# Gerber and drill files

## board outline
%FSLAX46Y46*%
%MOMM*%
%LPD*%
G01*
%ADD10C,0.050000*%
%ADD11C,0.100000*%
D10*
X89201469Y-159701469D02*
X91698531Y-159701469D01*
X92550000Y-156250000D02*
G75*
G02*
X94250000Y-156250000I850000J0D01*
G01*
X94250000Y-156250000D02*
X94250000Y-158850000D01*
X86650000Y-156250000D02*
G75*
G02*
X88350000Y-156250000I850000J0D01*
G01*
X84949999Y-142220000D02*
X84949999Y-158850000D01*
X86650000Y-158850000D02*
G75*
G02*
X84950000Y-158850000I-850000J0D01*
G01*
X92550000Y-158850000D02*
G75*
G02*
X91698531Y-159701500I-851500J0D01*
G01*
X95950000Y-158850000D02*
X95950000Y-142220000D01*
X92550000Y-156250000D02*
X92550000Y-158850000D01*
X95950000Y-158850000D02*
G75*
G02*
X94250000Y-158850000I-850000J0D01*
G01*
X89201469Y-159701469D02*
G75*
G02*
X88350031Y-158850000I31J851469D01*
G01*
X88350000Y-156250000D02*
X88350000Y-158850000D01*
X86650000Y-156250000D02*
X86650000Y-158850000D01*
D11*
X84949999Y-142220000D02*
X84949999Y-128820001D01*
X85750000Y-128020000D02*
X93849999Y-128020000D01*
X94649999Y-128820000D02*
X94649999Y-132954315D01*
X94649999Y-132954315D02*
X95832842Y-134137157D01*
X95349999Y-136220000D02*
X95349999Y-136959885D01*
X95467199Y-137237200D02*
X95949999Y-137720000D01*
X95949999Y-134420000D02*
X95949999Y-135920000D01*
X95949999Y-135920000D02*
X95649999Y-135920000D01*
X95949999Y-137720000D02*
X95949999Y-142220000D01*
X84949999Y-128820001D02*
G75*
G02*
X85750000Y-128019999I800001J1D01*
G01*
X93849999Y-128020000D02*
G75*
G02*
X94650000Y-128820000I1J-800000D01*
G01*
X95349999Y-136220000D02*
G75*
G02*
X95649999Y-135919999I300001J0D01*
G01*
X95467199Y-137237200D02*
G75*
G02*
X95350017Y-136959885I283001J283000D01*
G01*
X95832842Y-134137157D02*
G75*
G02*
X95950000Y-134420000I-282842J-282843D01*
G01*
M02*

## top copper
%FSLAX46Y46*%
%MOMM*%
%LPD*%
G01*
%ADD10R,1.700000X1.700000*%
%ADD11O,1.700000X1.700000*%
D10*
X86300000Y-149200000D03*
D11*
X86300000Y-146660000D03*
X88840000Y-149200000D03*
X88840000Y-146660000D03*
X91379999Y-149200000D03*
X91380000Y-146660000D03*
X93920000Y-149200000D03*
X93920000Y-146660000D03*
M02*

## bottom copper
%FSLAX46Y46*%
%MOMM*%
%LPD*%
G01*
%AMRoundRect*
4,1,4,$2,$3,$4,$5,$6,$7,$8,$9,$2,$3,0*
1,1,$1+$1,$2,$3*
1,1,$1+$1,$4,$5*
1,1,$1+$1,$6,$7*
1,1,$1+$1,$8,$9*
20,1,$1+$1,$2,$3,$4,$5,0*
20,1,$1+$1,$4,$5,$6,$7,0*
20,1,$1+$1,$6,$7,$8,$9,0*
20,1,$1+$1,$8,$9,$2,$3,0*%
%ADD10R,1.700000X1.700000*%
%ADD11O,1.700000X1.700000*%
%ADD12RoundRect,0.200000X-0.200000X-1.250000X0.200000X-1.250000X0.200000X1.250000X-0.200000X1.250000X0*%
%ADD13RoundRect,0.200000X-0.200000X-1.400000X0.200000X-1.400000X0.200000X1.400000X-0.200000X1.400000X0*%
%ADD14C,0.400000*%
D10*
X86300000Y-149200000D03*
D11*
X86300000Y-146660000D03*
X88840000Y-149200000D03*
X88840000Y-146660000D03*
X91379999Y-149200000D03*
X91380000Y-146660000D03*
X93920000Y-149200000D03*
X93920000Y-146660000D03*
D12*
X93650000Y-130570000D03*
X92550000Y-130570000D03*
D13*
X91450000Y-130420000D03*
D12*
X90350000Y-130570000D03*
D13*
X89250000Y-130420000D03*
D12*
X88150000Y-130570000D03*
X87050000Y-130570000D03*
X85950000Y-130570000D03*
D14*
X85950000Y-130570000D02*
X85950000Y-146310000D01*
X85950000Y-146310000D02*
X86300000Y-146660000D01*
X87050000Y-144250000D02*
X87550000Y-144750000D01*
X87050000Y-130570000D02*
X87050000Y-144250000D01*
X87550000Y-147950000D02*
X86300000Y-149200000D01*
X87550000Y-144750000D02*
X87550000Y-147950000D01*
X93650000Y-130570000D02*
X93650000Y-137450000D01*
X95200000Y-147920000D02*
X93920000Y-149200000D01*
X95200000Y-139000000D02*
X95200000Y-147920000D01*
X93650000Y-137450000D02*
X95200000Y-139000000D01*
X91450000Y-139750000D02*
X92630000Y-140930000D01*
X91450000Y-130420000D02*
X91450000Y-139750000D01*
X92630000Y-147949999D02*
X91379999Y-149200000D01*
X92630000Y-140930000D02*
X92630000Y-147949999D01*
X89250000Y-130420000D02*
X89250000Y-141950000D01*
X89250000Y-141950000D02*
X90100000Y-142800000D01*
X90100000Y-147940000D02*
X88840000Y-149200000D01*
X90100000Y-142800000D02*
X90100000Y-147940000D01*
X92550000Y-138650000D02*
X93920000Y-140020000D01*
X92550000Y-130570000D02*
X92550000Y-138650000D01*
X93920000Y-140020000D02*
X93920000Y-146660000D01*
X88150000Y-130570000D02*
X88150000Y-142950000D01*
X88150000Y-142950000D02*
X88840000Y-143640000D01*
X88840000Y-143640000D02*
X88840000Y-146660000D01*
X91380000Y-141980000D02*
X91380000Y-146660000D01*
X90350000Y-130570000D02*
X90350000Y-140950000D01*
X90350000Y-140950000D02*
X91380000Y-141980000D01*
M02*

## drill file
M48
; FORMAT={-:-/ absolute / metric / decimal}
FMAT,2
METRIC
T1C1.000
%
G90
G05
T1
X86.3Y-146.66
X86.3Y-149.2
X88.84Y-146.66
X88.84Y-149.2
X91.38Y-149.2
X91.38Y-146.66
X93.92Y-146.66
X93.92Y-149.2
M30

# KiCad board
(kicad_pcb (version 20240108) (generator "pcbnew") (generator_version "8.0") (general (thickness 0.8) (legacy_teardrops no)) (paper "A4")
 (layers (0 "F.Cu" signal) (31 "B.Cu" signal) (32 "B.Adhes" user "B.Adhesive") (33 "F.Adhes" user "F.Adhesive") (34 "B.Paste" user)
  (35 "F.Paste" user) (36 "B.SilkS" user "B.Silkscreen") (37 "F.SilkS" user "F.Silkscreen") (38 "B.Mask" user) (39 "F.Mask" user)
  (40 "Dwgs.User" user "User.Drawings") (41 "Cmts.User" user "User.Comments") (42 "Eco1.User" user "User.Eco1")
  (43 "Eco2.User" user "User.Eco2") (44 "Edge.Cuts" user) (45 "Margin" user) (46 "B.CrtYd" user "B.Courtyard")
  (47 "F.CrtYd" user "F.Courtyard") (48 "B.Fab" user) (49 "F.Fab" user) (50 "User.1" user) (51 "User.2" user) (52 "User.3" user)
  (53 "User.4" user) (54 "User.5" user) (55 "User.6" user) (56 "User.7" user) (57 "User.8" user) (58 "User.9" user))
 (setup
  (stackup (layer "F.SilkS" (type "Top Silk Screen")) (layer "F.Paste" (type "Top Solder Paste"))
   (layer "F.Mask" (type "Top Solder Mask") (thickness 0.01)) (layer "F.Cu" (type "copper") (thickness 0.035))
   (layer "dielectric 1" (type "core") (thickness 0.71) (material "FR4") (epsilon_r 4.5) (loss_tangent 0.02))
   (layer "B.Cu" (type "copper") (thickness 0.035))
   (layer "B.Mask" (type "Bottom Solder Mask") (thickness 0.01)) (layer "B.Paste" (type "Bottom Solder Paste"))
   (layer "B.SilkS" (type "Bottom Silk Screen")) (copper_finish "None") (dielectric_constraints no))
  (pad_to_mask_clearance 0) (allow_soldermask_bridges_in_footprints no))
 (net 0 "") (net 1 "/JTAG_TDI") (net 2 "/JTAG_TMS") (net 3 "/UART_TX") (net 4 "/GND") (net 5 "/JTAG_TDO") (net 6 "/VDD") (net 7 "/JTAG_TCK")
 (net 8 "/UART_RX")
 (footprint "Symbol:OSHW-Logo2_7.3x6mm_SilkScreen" (layer "F.Cu") (at 92.35 137.4 90)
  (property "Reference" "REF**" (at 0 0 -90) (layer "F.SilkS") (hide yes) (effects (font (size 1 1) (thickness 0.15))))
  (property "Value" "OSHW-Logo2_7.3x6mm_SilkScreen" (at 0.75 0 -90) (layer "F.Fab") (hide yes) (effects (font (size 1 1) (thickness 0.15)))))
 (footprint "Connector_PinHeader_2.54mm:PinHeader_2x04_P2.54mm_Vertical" (layer "F.Cu") (at 86.3 149.2 90)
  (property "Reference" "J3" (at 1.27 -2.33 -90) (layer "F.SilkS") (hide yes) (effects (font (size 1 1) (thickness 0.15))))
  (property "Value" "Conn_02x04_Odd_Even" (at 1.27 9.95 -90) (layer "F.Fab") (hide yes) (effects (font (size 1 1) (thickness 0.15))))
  (pad "1" thru_hole rect (at 0 0 90) (size 1.7 1.7) (drill 1) (layers "*.Cu" "*.Mask") (remove_unused_layers no) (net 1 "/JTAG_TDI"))
  (pad "2" thru_hole oval (at 2.54 0 90) (size 1.7 1.7) (drill 1) (layers "*.Cu" "*.Mask") (remove_unused_layers no) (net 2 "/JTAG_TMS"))
  (pad "3" thru_hole oval (at 0 2.54 90) (size 1.7 1.7) (drill 1) (layers "*.Cu" "*.Mask") (remove_unused_layers no) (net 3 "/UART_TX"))
  (pad "4" thru_hole oval (at 2.54 2.54 90) (size 1.7 1.7) (drill 1) (layers "*.Cu" "*.Mask") (remove_unused_layers no) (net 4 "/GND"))
  (pad "5" thru_hole oval (at 0 5.079999 90) (size 1.7 1.7) (drill 1) (layers "*.Cu" "*.Mask") (remove_unused_layers no) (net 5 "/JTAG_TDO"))
  (pad "6" thru_hole oval (at 2.54 5.08 90) (size 1.7 1.7) (drill 1) (layers "*.Cu" "*.Mask") (remove_unused_layers no) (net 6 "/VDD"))
  (pad "7" thru_hole oval (at 0 7.62 90) (size 1.7 1.7) (drill 1) (layers "*.Cu" "*.Mask") (remove_unused_layers no) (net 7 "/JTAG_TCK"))
  (pad "8" thru_hole oval (at 2.54 7.62 90) (size 1.7 1.7) (drill 1) (layers "*.Cu" "*.Mask") (remove_unused_layers no) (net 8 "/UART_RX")))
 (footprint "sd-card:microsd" (layer "F.Cu") (at 84.65 127.72)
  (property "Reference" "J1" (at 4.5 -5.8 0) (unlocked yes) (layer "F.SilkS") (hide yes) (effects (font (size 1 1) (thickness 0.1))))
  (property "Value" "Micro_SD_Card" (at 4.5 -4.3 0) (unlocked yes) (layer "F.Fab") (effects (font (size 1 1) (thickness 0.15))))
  (fp_line (start 0.299999 14.5) (end 0.299999 1.100001) (stroke (width 0.1) (type default)) (layer "Edge.Cuts"))
  (fp_line (start 1.1 0.3) (end 9.199999 0.3) (stroke (width 0.1) (type default)) (layer "Edge.Cuts"))
  (fp_line (start 9.999999 1.1) (end 9.999999 5.234315) (stroke (width 0.1) (type default)) (layer "Edge.Cuts"))
  (fp_line (start 9.999999 5.234315) (end 11.182842 6.417157) (stroke (width 0.1) (type default)) (layer "Edge.Cuts"))
  (fp_line (start 10.699999 8.5) (end 10.699999 9.239885) (stroke (width 0.1) (type default)) (layer "Edge.Cuts"))
  (fp_line (start 10.817199 9.5172) (end 11.299999 10) (stroke (width 0.1) (type default)) (layer "Edge.Cuts"))
  (fp_line (start 11.299999 6.7) (end 11.299999 8.2) (stroke (width 0.1) (type default)) (layer "Edge.Cuts"))
  (fp_line (start 11.299999 8.2) (end 10.999999 8.2) (stroke (width 0.1) (type default)) (layer "Edge.Cuts"))
  (fp_line (start 11.299999 10) (end 11.299999 14.5) (stroke (width 0.1) (type default)) (layer "Edge.Cuts"))
  (fp_arc (start 0.299999 1.100001) (mid 0.534314 0.534314) (end 1.1 0.3) (stroke (width 0.1) (type default)) (layer "Edge.Cuts"))
  (fp_arc (start 9.199999 0.3) (mid 9.765685 0.534314) (end 9.999999 1.1) (stroke (width 0.1) (type default)) (layer "Edge.Cuts"))
  (fp_arc (start 10.699999 8.5) (mid 10.787867 8.287868) (end 10.999999 8.2) (stroke (width 0.1) (type default)) (layer "Edge.Cuts"))
  (fp_arc (start 10.817199 9.5172) (mid 10.731528 9.389981) (end 10.699999 9.239885) (stroke (width 0.1) (type default)) (layer "Edge.Cuts"))
  (fp_arc (start 11.182842 6.417157) (mid 11.269551 6.546926) (end 11.299999 6.7) (stroke (width 0.1) (type default)) (layer "Edge.Cuts"))
  (pad "1" smd roundrect (at 9 2.85) (size 0.8 2.9) (layers "B.Cu" "B.Paste" "B.Mask") (roundrect_rratio 0.25) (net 7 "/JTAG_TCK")
   (thermal_bridge_angle 45))
  (pad "2" smd roundrect (at 7.9 2.85) (size 0.8 2.9) (layers "B.Cu" "B.Paste" "B.Mask") (roundrect_rratio 0.25) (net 8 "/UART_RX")
   (thermal_bridge_angle 45))
  (pad "3" smd roundrect (at 6.8 2.7) (size 0.8 3.2) (layers "B.Cu" "B.Paste" "B.Mask") (roundrect_rratio 0.25) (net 5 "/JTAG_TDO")
   (thermal_bridge_angle 45))
  (pad "4" smd roundrect (at 5.7 2.85) (size 0.8 2.9) (layers "B.Cu" "B.Paste" "B.Mask") (roundrect_rratio 0.25) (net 6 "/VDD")
   (thermal_bridge_angle 45))
  (pad "5" smd roundrect (at 4.6 2.7) (size 0.8 3.2) (layers "B.Cu" "B.Paste" "B.Mask") (roundrect_rratio 0.25) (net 3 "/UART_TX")
   (thermal_bridge_angle 45))
  (pad "6" smd roundrect (at 3.5 2.85) (size 0.8 2.9) (layers "B.Cu" "B.Paste" "B.Mask") (roundrect_rratio 0.25) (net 4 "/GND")
   (thermal_bridge_angle 45))
  (pad "7" smd roundrect (at 2.4 2.85) (size 0.8 2.9) (layers "B.Cu" "B.Paste" "B.Mask") (roundrect_rratio 0.25) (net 1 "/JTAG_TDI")
   (thermal_bridge_angle 45))
  (pad "8" smd roundrect (at 1.3 2.85) (size 0.8 2.9) (layers "B.Cu" "B.Paste" "B.Mask") (roundrect_rratio 0.25) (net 2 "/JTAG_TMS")
   (thermal_bridge_angle 45)))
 (gr_line (start 89.201469 159.701469) (end 91.698531 159.701469) (stroke (width 0.05) (type default)) (layer "Edge.Cuts"))
 (gr_arc (start 92.55 156.25) (mid 93.4 155.4) (end 94.25 156.25) (stroke (width 0.05) (type default)) (layer "Edge.Cuts"))
 (gr_line (start 94.25 156.25) (end 94.25 158.85) (stroke (width 0.05) (type default)) (layer "Edge.Cuts"))
 (gr_arc (start 86.65 156.25) (mid 87.5 155.4) (end 88.35 156.25) (stroke (width 0.05) (type default)) (layer "Edge.Cuts"))
 (gr_line (start 84.949999 142.22) (end 84.949999 158.85) (stroke (width 0.05) (type default)) (layer "Edge.Cuts"))
 (gr_arc (start 86.65 158.85) (mid 85.8 159.7) (end 84.95 158.85) (stroke (width 0.05) (type default)) (layer "Edge.Cuts"))
 (gr_arc (start 92.55 158.85) (mid 92.300611 159.45208) (end 91.698531 159.701469) (stroke (width 0.05) (type default)) (layer "Edge.Cuts"))
 (gr_line (start 95.95 158.85) (end 95.95 142.22) (stroke (width 0.05) (type default)) (layer "Edge.Cuts"))
 (gr_line (start 92.55 156.25) (end 92.55 158.85) (stroke (width 0.05) (type default)) (layer "Edge.Cuts"))
 (gr_arc (start 95.95 158.85) (mid 95.1 159.7) (end 94.25 158.85) (stroke (width 0.05) (type default)) (layer "Edge.Cuts"))
 (gr_arc (start 89.201469 159.701469) (mid 88.599389 159.45208) (end 88.35 158.85) (stroke (width 0.05) (type default)) (layer "Edge.Cuts"))
 (gr_line (start 88.35 156.25) (end 88.35 158.85) (stroke (width 0.05) (type default)) (layer "Edge.Cuts"))
 (gr_line (start 86.65 156.25) (end 86.65 158.85) (stroke (width 0.05) (type default)) (layer "Edge.Cuts"))
 (segment (start 85.95 130.57) (end 85.95 146.31) (width 0.4) (layer "B.Cu") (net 2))
 (segment (start 85.95 146.31) (end 86.3 146.66) (width 0.4) (layer "B.Cu") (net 2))
 (segment (start 87.05 144.25) (end 87.55 144.75) (width 0.4) (layer "B.Cu") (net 1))
 (segment (start 87.05 130.57) (end 87.05 144.25) (width 0.4) (layer "B.Cu") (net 1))
 (segment (start 87.55 147.95) (end 86.3 149.2) (width 0.4) (layer "B.Cu") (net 1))
 (segment (start 87.55 144.75) (end 87.55 147.95) (width 0.4) (layer "B.Cu") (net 1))
 (segment (start 93.65 130.57) (end 93.65 137.45) (width 0.4) (layer "B.Cu") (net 7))
 (segment (start 95.2 147.92) (end 93.92 149.2) (width 0.4) (layer "B.Cu") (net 7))
 (segment (start 95.2 139) (end 95.2 147.92) (width 0.4) (layer "B.Cu") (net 7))
 (segment (start 93.65 137.45) (end 95.2 139) (width 0.4) (layer "B.Cu") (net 7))
 (segment (start 91.45 139.75) (end 92.63 140.93) (width 0.4) (layer "B.Cu") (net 5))
 (segment (start 91.45 130.42) (end 91.45 139.75) (width 0.4) (layer "B.Cu") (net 5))
 (segment (start 92.63 147.949999) (end 91.379999 149.2) (width 0.4) (layer "B.Cu") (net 5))
 (segment (start 92.63 140.93) (end 92.63 147.949999) (width 0.4) (layer "B.Cu") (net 5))
 (segment (start 89.25 130.42) (end 89.25 141.95) (width 0.4) (layer "B.Cu") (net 3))
 (segment (start 89.25 141.95) (end 90.1 142.8) (width 0.4) (layer "B.Cu") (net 3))
 (segment (start 90.1 147.94) (end 88.84 149.2) (width 0.4) (layer "B.Cu") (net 3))
 (segment (start 90.1 142.8) (end 90.1 147.94) (width 0.4) (layer "B.Cu") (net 3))
 (segment (start 92.55 138.65) (end 93.92 140.02) (width 0.4) (layer "B.Cu") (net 8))
 (segment (start 92.55 130.57) (end 92.55 138.65) (width 0.4) (layer "B.Cu") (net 8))
 (segment (start 93.92 140.02) (end 93.92 146.66) (width 0.4) (layer "B.Cu") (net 8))
 (segment (start 88.15 130.57) (end 88.15 142.95) (width 0.4) (layer "B.Cu") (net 4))
 (segment (start 88.15 142.95) (end 88.84 143.64) (width 0.4) (layer "B.Cu") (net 4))
 (segment (start 88.84 143.64) (end 88.84 146.66) (width 0.4) (layer "B.Cu") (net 4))
 (segment (start 91.38 141.98) (end 91.38 146.66) (width 0.4) (layer "B.Cu") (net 6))
 (segment (start 90.35 130.57) (end 90.35 140.95) (width 0.4) (layer "B.Cu") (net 6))
 (segment (start 90.35 140.95) (end 91.38 141.98) (width 0.4) (layer "B.Cu") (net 6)))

